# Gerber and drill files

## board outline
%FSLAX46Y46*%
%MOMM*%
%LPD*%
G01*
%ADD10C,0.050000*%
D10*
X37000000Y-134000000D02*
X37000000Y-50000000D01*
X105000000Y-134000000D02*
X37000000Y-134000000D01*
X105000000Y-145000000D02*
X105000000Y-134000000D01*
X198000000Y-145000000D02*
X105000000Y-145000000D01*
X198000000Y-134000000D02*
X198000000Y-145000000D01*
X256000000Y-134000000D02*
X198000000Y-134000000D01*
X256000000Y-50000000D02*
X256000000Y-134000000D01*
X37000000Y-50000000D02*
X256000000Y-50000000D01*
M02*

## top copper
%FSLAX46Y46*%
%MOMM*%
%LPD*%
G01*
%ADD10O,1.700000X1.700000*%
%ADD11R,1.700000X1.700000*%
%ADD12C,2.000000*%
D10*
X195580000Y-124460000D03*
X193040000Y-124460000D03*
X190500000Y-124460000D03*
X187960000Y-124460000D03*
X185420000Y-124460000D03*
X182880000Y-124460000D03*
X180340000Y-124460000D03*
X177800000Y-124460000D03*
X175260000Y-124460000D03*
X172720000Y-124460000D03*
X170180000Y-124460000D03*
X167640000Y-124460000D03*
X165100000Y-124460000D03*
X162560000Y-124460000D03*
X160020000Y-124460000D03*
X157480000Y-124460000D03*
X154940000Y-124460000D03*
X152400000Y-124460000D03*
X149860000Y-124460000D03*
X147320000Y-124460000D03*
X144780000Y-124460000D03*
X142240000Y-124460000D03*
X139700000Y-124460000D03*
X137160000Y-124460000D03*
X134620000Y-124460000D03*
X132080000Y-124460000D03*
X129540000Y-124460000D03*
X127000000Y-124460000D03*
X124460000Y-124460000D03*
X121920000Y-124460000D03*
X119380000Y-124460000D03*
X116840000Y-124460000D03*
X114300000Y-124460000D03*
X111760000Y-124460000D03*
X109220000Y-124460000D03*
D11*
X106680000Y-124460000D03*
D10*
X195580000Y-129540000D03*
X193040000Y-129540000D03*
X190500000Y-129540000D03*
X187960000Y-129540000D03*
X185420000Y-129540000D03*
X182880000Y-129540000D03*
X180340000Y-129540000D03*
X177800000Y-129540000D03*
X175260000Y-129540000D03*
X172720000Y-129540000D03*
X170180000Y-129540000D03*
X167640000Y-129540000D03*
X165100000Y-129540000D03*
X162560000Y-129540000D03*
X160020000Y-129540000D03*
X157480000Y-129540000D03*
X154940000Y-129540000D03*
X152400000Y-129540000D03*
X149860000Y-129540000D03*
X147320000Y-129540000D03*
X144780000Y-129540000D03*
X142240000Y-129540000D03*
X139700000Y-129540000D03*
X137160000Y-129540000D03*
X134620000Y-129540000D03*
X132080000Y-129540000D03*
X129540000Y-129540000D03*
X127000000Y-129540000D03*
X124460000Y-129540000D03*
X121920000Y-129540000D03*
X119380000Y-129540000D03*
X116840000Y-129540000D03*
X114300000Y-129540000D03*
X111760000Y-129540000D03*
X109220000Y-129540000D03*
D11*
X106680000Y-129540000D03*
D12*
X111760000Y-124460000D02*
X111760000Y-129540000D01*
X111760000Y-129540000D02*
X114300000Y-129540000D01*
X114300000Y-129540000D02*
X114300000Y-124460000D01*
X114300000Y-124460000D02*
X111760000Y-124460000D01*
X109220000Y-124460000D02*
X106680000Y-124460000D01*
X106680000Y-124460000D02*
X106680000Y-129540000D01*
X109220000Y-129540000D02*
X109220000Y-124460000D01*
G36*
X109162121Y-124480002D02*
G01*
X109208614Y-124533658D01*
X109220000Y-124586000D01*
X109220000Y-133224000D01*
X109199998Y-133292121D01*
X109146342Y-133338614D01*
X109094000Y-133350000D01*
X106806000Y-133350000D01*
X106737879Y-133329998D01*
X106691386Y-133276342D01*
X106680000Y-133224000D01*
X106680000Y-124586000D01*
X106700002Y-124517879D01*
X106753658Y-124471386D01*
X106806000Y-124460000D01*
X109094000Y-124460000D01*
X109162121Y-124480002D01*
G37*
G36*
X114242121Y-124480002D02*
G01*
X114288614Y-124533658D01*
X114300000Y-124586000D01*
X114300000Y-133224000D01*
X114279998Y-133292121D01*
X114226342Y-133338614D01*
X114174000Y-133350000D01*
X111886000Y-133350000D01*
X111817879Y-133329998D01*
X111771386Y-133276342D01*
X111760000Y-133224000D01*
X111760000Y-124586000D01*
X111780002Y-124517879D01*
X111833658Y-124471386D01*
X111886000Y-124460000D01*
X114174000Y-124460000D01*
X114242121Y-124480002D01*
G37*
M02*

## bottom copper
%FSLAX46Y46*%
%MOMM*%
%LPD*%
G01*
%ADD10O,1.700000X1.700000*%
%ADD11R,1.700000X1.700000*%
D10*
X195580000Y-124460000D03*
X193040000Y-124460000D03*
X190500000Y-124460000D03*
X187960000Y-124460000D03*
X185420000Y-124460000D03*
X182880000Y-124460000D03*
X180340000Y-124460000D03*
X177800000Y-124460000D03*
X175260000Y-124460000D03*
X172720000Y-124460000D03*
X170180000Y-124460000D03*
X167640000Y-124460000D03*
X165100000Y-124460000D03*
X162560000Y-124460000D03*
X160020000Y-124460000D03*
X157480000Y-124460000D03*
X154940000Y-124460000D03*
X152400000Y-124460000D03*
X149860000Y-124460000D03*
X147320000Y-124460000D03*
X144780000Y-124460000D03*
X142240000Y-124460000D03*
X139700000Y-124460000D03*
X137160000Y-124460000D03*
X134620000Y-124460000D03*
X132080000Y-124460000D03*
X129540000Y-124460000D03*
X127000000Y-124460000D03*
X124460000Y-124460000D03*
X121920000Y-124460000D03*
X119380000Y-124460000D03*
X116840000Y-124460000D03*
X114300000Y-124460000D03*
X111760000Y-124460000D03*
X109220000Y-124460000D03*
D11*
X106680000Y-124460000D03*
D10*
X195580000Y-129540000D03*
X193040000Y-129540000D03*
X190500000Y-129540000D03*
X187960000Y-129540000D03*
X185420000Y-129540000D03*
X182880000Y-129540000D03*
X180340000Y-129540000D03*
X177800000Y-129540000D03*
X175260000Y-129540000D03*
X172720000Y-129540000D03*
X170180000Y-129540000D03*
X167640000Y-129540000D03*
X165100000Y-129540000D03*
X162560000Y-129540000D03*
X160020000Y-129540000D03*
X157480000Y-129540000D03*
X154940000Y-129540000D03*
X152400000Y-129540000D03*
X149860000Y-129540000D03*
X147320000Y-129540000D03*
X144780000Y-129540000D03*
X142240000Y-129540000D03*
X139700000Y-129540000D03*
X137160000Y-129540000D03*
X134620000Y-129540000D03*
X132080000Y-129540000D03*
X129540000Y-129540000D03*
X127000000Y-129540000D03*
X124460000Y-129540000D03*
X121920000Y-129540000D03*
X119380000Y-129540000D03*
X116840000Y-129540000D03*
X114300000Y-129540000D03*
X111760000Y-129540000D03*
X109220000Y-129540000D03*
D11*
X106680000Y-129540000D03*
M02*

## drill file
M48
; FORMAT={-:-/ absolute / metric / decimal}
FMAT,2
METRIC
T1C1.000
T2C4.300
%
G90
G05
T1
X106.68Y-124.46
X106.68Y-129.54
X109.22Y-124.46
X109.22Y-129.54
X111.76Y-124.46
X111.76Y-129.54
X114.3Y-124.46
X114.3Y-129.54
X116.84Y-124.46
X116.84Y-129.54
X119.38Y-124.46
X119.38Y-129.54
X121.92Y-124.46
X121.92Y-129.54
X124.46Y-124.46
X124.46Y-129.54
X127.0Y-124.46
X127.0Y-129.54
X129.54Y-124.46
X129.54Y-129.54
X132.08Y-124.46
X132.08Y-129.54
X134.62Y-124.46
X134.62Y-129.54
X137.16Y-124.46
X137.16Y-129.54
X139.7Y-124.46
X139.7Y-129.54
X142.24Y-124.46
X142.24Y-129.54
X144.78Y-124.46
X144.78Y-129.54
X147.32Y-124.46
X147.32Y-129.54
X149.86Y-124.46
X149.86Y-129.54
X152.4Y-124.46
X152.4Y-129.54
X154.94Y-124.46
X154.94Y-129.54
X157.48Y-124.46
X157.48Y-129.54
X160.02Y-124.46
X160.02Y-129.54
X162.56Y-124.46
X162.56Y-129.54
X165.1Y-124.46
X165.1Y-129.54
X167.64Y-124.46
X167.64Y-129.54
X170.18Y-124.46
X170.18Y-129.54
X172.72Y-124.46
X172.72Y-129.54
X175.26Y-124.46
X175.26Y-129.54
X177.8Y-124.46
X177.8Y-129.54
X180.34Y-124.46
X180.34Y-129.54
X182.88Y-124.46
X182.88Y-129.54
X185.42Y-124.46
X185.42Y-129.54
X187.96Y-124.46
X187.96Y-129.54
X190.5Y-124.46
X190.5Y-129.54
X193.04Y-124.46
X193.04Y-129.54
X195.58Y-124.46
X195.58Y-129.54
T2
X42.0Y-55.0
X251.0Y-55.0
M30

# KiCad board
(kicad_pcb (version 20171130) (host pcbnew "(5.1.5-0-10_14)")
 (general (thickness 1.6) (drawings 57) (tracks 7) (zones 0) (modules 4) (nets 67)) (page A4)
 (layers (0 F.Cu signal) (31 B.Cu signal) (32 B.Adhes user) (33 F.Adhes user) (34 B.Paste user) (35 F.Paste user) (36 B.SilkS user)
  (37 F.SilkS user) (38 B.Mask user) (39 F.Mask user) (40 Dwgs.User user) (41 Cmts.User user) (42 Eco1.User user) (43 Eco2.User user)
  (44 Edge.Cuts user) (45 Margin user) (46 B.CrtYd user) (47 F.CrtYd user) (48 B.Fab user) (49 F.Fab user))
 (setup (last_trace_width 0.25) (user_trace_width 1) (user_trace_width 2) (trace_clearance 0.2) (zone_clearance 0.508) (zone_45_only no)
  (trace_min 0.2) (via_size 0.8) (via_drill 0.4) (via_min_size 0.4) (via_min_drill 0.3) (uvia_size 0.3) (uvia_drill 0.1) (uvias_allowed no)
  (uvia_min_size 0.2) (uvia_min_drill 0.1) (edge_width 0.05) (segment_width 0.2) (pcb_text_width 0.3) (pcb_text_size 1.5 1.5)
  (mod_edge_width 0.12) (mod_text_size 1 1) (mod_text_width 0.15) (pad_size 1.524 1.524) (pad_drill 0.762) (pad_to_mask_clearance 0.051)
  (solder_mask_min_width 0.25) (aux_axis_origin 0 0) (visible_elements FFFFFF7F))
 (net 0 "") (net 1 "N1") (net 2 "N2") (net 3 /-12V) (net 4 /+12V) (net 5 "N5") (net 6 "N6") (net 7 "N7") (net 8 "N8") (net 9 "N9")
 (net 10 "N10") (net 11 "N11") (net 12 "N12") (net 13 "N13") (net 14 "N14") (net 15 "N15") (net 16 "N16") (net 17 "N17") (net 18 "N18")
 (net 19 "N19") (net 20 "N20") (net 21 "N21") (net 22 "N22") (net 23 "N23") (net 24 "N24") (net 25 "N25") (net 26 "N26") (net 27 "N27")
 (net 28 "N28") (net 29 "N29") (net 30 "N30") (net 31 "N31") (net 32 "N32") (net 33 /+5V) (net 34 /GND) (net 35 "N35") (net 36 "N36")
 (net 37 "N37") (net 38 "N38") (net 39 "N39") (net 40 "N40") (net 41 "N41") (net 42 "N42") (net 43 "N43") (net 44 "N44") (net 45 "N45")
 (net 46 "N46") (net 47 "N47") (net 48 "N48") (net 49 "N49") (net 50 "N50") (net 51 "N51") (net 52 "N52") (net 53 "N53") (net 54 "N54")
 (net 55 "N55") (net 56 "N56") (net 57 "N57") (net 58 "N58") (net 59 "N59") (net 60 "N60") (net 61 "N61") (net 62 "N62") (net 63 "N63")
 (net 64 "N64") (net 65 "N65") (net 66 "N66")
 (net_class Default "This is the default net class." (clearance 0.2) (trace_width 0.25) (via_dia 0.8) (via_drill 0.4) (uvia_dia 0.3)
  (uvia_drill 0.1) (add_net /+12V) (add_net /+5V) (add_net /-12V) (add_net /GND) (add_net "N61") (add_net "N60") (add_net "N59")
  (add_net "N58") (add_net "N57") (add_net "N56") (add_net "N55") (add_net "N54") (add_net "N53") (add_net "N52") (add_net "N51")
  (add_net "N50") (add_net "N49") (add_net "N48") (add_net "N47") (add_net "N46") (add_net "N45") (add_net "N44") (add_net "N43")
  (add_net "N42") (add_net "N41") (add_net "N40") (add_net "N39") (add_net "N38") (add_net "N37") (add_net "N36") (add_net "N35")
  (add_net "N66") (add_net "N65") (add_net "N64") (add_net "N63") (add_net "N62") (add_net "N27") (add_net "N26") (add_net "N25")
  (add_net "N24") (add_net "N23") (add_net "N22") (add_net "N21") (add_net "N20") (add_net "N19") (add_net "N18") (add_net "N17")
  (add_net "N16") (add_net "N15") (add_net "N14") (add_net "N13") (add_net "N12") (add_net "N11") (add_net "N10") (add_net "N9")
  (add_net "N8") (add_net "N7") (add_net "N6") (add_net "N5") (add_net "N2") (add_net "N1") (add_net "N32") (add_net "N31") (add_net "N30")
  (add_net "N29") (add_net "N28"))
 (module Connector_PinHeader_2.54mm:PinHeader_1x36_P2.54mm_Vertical (layer F.Cu) (at 106.68 124.46 90)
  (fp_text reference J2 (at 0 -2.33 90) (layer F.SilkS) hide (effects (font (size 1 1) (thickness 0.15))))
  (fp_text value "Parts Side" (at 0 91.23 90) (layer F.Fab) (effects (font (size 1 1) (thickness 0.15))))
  (pad 36 thru_hole oval (at 0 88.9 90) (size 1.7 1.7) (drill 1) (layers *.Cu *.Mask) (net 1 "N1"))
  (pad 35 thru_hole oval (at 0 86.36 90) (size 1.7 1.7) (drill 1) (layers *.Cu *.Mask) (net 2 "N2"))
  (pad 34 thru_hole oval (at 0 83.82 90) (size 1.7 1.7) (drill 1) (layers *.Cu *.Mask) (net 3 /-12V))
  (pad 33 thru_hole oval (at 0 81.28 90) (size 1.7 1.7) (drill 1) (layers *.Cu *.Mask) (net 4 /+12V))
  (pad 32 thru_hole oval (at 0 78.74 90) (size 1.7 1.7) (drill 1) (layers *.Cu *.Mask) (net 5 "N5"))
  (pad 31 thru_hole oval (at 0 76.2 90) (size 1.7 1.7) (drill 1) (layers *.Cu *.Mask) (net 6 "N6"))
  (pad 30 thru_hole oval (at 0 73.66 90) (size 1.7 1.7) (drill 1) (layers *.Cu *.Mask) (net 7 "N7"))
  (pad 29 thru_hole oval (at 0 71.12 90) (size 1.7 1.7) (drill 1) (layers *.Cu *.Mask) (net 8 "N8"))
  (pad 28 thru_hole oval (at 0 68.58 90) (size 1.7 1.7) (drill 1) (layers *.Cu *.Mask) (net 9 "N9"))
  (pad 27 thru_hole oval (at 0 66.04 90) (size 1.7 1.7) (drill 1) (layers *.Cu *.Mask) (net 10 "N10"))
  (pad 26 thru_hole oval (at 0 63.5 90) (size 1.7 1.7) (drill 1) (layers *.Cu *.Mask) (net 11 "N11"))
  (pad 25 thru_hole oval (at 0 60.96 90) (size 1.7 1.7) (drill 1) (layers *.Cu *.Mask) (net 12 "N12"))
  (pad 24 thru_hole oval (at 0 58.42 90) (size 1.7 1.7) (drill 1) (layers *.Cu *.Mask) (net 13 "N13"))
  (pad 23 thru_hole oval (at 0 55.88 90) (size 1.7 1.7) (drill 1) (layers *.Cu *.Mask) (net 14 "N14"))
  (pad 22 thru_hole oval (at 0 53.34 90) (size 1.7 1.7) (drill 1) (layers *.Cu *.Mask) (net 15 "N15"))
  (pad 21 thru_hole oval (at 0 50.8 90) (size 1.7 1.7) (drill 1) (layers *.Cu *.Mask) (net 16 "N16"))
  (pad 20 thru_hole oval (at 0 48.26 90) (size 1.7 1.7) (drill 1) (layers *.Cu *.Mask) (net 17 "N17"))
  (pad 19 thru_hole oval (at 0 45.72 90) (size 1.7 1.7) (drill 1) (layers *.Cu *.Mask) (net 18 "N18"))
  (pad 18 thru_hole oval (at 0 43.18 90) (size 1.7 1.7) (drill 1) (layers *.Cu *.Mask) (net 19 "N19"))
  (pad 17 thru_hole oval (at 0 40.64 90) (size 1.7 1.7) (drill 1) (layers *.Cu *.Mask) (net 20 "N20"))
  (pad 16 thru_hole oval (at 0 38.1 90) (size 1.7 1.7) (drill 1) (layers *.Cu *.Mask) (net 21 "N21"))
  (pad 15 thru_hole oval (at 0 35.56 90) (size 1.7 1.7) (drill 1) (layers *.Cu *.Mask) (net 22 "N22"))
  (pad 14 thru_hole oval (at 0 33.02 90) (size 1.7 1.7) (drill 1) (layers *.Cu *.Mask) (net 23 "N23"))
  (pad 13 thru_hole oval (at 0 30.48 90) (size 1.7 1.7) (drill 1) (layers *.Cu *.Mask) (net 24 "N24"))
  (pad 12 thru_hole oval (at 0 27.94 90) (size 1.7 1.7) (drill 1) (layers *.Cu *.Mask) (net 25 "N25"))
  (pad 11 thru_hole oval (at 0 25.4 90) (size 1.7 1.7) (drill 1) (layers *.Cu *.Mask) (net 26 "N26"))
  (pad 10 thru_hole oval (at 0 22.86 90) (size 1.7 1.7) (drill 1) (layers *.Cu *.Mask) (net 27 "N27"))
  (pad 9 thru_hole oval (at 0 20.32 90) (size 1.7 1.7) (drill 1) (layers *.Cu *.Mask) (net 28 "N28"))
  (pad 8 thru_hole oval (at 0 17.78 90) (size 1.7 1.7) (drill 1) (layers *.Cu *.Mask) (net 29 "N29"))
  (pad 7 thru_hole oval (at 0 15.24 90) (size 1.7 1.7) (drill 1) (layers *.Cu *.Mask) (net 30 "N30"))
  (pad 6 thru_hole oval (at 0 12.7 90) (size 1.7 1.7) (drill 1) (layers *.Cu *.Mask) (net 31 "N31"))
  (pad 5 thru_hole oval (at 0 10.16 90) (size 1.7 1.7) (drill 1) (layers *.Cu *.Mask) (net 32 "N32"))
  (pad 4 thru_hole oval (at 0 7.62 90) (size 1.7 1.7) (drill 1) (layers *.Cu *.Mask) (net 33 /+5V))
  (pad 3 thru_hole oval (at 0 5.08 90) (size 1.7 1.7) (drill 1) (layers *.Cu *.Mask) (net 33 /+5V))
  (pad 2 thru_hole oval (at 0 2.54 90) (size 1.7 1.7) (drill 1) (layers *.Cu *.Mask) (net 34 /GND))
  (pad 1 thru_hole rect (at 0 0 90) (size 1.7 1.7) (drill 1) (layers *.Cu *.Mask) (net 34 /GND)))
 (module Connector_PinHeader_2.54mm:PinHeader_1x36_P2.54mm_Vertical (layer F.Cu) (at 106.68 129.54 90)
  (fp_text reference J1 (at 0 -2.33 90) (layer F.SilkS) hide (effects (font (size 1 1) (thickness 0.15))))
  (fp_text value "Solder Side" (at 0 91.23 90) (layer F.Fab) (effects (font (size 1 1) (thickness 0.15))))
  (pad 36 thru_hole oval (at 0 88.9 90) (size 1.7 1.7) (drill 1) (layers *.Cu *.Mask) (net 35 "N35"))
  (pad 35 thru_hole oval (at 0 86.36 90) (size 1.7 1.7) (drill 1) (layers *.Cu *.Mask) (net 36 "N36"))
  (pad 34 thru_hole oval (at 0 83.82 90) (size 1.7 1.7) (drill 1) (layers *.Cu *.Mask) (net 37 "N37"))
  (pad 33 thru_hole oval (at 0 81.28 90) (size 1.7 1.7) (drill 1) (layers *.Cu *.Mask) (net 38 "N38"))
  (pad 32 thru_hole oval (at 0 78.74 90) (size 1.7 1.7) (drill 1) (layers *.Cu *.Mask) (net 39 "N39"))
  (pad 31 thru_hole oval (at 0 76.2 90) (size 1.7 1.7) (drill 1) (layers *.Cu *.Mask) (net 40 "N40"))
  (pad 30 thru_hole oval (at 0 73.66 90) (size 1.7 1.7) (drill 1) (layers *.Cu *.Mask) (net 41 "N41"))
  (pad 29 thru_hole oval (at 0 71.12 90) (size 1.7 1.7) (drill 1) (layers *.Cu *.Mask) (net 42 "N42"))
  (pad 28 thru_hole oval (at 0 68.58 90) (size 1.7 1.7) (drill 1) (layers *.Cu *.Mask) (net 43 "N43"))
  (pad 27 thru_hole oval (at 0 66.04 90) (size 1.7 1.7) (drill 1) (layers *.Cu *.Mask) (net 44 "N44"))
  (pad 26 thru_hole oval (at 0 63.5 90) (size 1.7 1.7) (drill 1) (layers *.Cu *.Mask) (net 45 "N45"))
  (pad 25 thru_hole oval (at 0 60.96 90) (size 1.7 1.7) (drill 1) (layers *.Cu *.Mask) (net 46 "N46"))
  (pad 24 thru_hole oval (at 0 58.42 90) (size 1.7 1.7) (drill 1) (layers *.Cu *.Mask) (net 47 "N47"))
  (pad 23 thru_hole oval (at 0 55.88 90) (size 1.7 1.7) (drill 1) (layers *.Cu *.Mask) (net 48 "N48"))
  (pad 22 thru_hole oval (at 0 53.34 90) (size 1.7 1.7) (drill 1) (layers *.Cu *.Mask) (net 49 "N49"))
  (pad 21 thru_hole oval (at 0 50.8 90) (size 1.7 1.7) (drill 1) (layers *.Cu *.Mask) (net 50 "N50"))
  (pad 20 thru_hole oval (at 0 48.26 90) (size 1.7 1.7) (drill 1) (layers *.Cu *.Mask) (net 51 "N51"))
  (pad 19 thru_hole oval (at 0 45.72 90) (size 1.7 1.7) (drill 1) (layers *.Cu *.Mask) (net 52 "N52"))
  (pad 18 thru_hole oval (at 0 43.18 90) (size 1.7 1.7) (drill 1) (layers *.Cu *.Mask) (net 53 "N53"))
  (pad 17 thru_hole oval (at 0 40.64 90) (size 1.7 1.7) (drill 1) (layers *.Cu *.Mask) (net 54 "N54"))
  (pad 16 thru_hole oval (at 0 38.1 90) (size 1.7 1.7) (drill 1) (layers *.Cu *.Mask) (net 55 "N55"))
  (pad 15 thru_hole oval (at 0 35.56 90) (size 1.7 1.7) (drill 1) (layers *.Cu *.Mask) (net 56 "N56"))
  (pad 14 thru_hole oval (at 0 33.02 90) (size 1.7 1.7) (drill 1) (layers *.Cu *.Mask) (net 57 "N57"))
  (pad 13 thru_hole oval (at 0 30.48 90) (size 1.7 1.7) (drill 1) (layers *.Cu *.Mask) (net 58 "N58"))
  (pad 12 thru_hole oval (at 0 27.94 90) (size 1.7 1.7) (drill 1) (layers *.Cu *.Mask) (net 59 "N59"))
  (pad 11 thru_hole oval (at 0 25.4 90) (size 1.7 1.7) (drill 1) (layers *.Cu *.Mask) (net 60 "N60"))
  (pad 10 thru_hole oval (at 0 22.86 90) (size 1.7 1.7) (drill 1) (layers *.Cu *.Mask) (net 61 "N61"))
  (pad 9 thru_hole oval (at 0 20.32 90) (size 1.7 1.7) (drill 1) (layers *.Cu *.Mask) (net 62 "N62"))
  (pad 8 thru_hole oval (at 0 17.78 90) (size 1.7 1.7) (drill 1) (layers *.Cu *.Mask) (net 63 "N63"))
  (pad 7 thru_hole oval (at 0 15.24 90) (size 1.7 1.7) (drill 1) (layers *.Cu *.Mask) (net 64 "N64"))
  (pad 6 thru_hole oval (at 0 12.7 90) (size 1.7 1.7) (drill 1) (layers *.Cu *.Mask) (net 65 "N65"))
  (pad 5 thru_hole oval (at 0 10.16 90) (size 1.7 1.7) (drill 1) (layers *.Cu *.Mask) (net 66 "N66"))
  (pad 4 thru_hole oval (at 0 7.62 90) (size 1.7 1.7) (drill 1) (layers *.Cu *.Mask) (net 33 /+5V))
  (pad 3 thru_hole oval (at 0 5.08 90) (size 1.7 1.7) (drill 1) (layers *.Cu *.Mask) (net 33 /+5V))
  (pad 2 thru_hole oval (at 0 2.54 90) (size 1.7 1.7) (drill 1) (layers *.Cu *.Mask) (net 34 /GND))
  (pad 1 thru_hole rect (at 0 0 90) (size 1.7 1.7) (drill 1) (layers *.Cu *.Mask) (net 34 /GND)))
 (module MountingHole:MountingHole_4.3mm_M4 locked (layer F.Cu) (at 42 55)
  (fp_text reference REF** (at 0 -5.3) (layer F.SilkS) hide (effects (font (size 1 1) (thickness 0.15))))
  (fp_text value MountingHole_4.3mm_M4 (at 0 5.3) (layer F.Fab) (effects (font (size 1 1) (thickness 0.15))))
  (pad 1 np_thru_hole circle (at 0 0) (size 4.3 4.3) (drill 4.3) (layers *.Cu *.Mask)))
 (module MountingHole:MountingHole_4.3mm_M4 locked (layer F.Cu) (at 251 55)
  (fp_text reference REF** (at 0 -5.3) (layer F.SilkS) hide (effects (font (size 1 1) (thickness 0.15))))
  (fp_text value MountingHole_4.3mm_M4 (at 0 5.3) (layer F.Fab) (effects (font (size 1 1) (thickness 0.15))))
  (pad 1 np_thru_hole circle (at 0 0) (size 4.3 4.3) (drill 4.3) (layers *.Cu *.Mask)))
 (gr_line (start 37 134) (end 37 50) (layer Edge.Cuts) (width 0.05))
 (gr_line (start 105 134) (end 37 134) (layer Edge.Cuts) (width 0.05))
 (gr_line (start 105 145) (end 105 134) (layer Edge.Cuts) (width 0.05))
 (gr_line (start 198 145) (end 105 145) (layer Edge.Cuts) (width 0.05))
 (gr_line (start 198 134) (end 198 145) (layer Edge.Cuts) (width 0.05))
 (gr_line (start 256 134) (end 198 134) (layer Edge.Cuts) (width 0.05))
 (gr_line (start 256 50) (end 256 134) (layer Edge.Cuts) (width 0.05))
 (gr_line (start 37 50) (end 256 50) (layer Edge.Cuts) (width 0.05))
 (segment (start 111.76 124.46) (end 111.76 129.54) (width 2) (layer F.Cu) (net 33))
 (segment (start 111.76 129.54) (end 114.3 129.54) (width 2) (layer F.Cu) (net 33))
 (segment (start 114.3 129.54) (end 114.3 124.46) (width 2) (layer F.Cu) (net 33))
 (segment (start 114.3 124.46) (end 111.76 124.46) (width 2) (layer F.Cu) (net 33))
 (segment (start 109.22 124.46) (end 106.68 124.46) (width 2) (layer F.Cu) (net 34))
 (segment (start 106.68 124.46) (end 106.68 129.54) (width 2) (layer F.Cu) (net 34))
 (segment (start 109.22 129.54) (end 109.22 124.46) (width 2) (layer F.Cu) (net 34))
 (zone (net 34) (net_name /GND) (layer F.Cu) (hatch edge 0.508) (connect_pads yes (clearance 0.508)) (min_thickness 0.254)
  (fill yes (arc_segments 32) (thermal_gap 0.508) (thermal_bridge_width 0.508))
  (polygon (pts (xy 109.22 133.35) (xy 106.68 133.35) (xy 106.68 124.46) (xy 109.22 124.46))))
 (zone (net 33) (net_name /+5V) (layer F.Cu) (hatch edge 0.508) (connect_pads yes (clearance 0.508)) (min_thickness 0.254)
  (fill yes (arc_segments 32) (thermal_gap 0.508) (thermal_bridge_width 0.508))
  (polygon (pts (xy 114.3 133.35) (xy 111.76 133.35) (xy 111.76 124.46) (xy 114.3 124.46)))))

